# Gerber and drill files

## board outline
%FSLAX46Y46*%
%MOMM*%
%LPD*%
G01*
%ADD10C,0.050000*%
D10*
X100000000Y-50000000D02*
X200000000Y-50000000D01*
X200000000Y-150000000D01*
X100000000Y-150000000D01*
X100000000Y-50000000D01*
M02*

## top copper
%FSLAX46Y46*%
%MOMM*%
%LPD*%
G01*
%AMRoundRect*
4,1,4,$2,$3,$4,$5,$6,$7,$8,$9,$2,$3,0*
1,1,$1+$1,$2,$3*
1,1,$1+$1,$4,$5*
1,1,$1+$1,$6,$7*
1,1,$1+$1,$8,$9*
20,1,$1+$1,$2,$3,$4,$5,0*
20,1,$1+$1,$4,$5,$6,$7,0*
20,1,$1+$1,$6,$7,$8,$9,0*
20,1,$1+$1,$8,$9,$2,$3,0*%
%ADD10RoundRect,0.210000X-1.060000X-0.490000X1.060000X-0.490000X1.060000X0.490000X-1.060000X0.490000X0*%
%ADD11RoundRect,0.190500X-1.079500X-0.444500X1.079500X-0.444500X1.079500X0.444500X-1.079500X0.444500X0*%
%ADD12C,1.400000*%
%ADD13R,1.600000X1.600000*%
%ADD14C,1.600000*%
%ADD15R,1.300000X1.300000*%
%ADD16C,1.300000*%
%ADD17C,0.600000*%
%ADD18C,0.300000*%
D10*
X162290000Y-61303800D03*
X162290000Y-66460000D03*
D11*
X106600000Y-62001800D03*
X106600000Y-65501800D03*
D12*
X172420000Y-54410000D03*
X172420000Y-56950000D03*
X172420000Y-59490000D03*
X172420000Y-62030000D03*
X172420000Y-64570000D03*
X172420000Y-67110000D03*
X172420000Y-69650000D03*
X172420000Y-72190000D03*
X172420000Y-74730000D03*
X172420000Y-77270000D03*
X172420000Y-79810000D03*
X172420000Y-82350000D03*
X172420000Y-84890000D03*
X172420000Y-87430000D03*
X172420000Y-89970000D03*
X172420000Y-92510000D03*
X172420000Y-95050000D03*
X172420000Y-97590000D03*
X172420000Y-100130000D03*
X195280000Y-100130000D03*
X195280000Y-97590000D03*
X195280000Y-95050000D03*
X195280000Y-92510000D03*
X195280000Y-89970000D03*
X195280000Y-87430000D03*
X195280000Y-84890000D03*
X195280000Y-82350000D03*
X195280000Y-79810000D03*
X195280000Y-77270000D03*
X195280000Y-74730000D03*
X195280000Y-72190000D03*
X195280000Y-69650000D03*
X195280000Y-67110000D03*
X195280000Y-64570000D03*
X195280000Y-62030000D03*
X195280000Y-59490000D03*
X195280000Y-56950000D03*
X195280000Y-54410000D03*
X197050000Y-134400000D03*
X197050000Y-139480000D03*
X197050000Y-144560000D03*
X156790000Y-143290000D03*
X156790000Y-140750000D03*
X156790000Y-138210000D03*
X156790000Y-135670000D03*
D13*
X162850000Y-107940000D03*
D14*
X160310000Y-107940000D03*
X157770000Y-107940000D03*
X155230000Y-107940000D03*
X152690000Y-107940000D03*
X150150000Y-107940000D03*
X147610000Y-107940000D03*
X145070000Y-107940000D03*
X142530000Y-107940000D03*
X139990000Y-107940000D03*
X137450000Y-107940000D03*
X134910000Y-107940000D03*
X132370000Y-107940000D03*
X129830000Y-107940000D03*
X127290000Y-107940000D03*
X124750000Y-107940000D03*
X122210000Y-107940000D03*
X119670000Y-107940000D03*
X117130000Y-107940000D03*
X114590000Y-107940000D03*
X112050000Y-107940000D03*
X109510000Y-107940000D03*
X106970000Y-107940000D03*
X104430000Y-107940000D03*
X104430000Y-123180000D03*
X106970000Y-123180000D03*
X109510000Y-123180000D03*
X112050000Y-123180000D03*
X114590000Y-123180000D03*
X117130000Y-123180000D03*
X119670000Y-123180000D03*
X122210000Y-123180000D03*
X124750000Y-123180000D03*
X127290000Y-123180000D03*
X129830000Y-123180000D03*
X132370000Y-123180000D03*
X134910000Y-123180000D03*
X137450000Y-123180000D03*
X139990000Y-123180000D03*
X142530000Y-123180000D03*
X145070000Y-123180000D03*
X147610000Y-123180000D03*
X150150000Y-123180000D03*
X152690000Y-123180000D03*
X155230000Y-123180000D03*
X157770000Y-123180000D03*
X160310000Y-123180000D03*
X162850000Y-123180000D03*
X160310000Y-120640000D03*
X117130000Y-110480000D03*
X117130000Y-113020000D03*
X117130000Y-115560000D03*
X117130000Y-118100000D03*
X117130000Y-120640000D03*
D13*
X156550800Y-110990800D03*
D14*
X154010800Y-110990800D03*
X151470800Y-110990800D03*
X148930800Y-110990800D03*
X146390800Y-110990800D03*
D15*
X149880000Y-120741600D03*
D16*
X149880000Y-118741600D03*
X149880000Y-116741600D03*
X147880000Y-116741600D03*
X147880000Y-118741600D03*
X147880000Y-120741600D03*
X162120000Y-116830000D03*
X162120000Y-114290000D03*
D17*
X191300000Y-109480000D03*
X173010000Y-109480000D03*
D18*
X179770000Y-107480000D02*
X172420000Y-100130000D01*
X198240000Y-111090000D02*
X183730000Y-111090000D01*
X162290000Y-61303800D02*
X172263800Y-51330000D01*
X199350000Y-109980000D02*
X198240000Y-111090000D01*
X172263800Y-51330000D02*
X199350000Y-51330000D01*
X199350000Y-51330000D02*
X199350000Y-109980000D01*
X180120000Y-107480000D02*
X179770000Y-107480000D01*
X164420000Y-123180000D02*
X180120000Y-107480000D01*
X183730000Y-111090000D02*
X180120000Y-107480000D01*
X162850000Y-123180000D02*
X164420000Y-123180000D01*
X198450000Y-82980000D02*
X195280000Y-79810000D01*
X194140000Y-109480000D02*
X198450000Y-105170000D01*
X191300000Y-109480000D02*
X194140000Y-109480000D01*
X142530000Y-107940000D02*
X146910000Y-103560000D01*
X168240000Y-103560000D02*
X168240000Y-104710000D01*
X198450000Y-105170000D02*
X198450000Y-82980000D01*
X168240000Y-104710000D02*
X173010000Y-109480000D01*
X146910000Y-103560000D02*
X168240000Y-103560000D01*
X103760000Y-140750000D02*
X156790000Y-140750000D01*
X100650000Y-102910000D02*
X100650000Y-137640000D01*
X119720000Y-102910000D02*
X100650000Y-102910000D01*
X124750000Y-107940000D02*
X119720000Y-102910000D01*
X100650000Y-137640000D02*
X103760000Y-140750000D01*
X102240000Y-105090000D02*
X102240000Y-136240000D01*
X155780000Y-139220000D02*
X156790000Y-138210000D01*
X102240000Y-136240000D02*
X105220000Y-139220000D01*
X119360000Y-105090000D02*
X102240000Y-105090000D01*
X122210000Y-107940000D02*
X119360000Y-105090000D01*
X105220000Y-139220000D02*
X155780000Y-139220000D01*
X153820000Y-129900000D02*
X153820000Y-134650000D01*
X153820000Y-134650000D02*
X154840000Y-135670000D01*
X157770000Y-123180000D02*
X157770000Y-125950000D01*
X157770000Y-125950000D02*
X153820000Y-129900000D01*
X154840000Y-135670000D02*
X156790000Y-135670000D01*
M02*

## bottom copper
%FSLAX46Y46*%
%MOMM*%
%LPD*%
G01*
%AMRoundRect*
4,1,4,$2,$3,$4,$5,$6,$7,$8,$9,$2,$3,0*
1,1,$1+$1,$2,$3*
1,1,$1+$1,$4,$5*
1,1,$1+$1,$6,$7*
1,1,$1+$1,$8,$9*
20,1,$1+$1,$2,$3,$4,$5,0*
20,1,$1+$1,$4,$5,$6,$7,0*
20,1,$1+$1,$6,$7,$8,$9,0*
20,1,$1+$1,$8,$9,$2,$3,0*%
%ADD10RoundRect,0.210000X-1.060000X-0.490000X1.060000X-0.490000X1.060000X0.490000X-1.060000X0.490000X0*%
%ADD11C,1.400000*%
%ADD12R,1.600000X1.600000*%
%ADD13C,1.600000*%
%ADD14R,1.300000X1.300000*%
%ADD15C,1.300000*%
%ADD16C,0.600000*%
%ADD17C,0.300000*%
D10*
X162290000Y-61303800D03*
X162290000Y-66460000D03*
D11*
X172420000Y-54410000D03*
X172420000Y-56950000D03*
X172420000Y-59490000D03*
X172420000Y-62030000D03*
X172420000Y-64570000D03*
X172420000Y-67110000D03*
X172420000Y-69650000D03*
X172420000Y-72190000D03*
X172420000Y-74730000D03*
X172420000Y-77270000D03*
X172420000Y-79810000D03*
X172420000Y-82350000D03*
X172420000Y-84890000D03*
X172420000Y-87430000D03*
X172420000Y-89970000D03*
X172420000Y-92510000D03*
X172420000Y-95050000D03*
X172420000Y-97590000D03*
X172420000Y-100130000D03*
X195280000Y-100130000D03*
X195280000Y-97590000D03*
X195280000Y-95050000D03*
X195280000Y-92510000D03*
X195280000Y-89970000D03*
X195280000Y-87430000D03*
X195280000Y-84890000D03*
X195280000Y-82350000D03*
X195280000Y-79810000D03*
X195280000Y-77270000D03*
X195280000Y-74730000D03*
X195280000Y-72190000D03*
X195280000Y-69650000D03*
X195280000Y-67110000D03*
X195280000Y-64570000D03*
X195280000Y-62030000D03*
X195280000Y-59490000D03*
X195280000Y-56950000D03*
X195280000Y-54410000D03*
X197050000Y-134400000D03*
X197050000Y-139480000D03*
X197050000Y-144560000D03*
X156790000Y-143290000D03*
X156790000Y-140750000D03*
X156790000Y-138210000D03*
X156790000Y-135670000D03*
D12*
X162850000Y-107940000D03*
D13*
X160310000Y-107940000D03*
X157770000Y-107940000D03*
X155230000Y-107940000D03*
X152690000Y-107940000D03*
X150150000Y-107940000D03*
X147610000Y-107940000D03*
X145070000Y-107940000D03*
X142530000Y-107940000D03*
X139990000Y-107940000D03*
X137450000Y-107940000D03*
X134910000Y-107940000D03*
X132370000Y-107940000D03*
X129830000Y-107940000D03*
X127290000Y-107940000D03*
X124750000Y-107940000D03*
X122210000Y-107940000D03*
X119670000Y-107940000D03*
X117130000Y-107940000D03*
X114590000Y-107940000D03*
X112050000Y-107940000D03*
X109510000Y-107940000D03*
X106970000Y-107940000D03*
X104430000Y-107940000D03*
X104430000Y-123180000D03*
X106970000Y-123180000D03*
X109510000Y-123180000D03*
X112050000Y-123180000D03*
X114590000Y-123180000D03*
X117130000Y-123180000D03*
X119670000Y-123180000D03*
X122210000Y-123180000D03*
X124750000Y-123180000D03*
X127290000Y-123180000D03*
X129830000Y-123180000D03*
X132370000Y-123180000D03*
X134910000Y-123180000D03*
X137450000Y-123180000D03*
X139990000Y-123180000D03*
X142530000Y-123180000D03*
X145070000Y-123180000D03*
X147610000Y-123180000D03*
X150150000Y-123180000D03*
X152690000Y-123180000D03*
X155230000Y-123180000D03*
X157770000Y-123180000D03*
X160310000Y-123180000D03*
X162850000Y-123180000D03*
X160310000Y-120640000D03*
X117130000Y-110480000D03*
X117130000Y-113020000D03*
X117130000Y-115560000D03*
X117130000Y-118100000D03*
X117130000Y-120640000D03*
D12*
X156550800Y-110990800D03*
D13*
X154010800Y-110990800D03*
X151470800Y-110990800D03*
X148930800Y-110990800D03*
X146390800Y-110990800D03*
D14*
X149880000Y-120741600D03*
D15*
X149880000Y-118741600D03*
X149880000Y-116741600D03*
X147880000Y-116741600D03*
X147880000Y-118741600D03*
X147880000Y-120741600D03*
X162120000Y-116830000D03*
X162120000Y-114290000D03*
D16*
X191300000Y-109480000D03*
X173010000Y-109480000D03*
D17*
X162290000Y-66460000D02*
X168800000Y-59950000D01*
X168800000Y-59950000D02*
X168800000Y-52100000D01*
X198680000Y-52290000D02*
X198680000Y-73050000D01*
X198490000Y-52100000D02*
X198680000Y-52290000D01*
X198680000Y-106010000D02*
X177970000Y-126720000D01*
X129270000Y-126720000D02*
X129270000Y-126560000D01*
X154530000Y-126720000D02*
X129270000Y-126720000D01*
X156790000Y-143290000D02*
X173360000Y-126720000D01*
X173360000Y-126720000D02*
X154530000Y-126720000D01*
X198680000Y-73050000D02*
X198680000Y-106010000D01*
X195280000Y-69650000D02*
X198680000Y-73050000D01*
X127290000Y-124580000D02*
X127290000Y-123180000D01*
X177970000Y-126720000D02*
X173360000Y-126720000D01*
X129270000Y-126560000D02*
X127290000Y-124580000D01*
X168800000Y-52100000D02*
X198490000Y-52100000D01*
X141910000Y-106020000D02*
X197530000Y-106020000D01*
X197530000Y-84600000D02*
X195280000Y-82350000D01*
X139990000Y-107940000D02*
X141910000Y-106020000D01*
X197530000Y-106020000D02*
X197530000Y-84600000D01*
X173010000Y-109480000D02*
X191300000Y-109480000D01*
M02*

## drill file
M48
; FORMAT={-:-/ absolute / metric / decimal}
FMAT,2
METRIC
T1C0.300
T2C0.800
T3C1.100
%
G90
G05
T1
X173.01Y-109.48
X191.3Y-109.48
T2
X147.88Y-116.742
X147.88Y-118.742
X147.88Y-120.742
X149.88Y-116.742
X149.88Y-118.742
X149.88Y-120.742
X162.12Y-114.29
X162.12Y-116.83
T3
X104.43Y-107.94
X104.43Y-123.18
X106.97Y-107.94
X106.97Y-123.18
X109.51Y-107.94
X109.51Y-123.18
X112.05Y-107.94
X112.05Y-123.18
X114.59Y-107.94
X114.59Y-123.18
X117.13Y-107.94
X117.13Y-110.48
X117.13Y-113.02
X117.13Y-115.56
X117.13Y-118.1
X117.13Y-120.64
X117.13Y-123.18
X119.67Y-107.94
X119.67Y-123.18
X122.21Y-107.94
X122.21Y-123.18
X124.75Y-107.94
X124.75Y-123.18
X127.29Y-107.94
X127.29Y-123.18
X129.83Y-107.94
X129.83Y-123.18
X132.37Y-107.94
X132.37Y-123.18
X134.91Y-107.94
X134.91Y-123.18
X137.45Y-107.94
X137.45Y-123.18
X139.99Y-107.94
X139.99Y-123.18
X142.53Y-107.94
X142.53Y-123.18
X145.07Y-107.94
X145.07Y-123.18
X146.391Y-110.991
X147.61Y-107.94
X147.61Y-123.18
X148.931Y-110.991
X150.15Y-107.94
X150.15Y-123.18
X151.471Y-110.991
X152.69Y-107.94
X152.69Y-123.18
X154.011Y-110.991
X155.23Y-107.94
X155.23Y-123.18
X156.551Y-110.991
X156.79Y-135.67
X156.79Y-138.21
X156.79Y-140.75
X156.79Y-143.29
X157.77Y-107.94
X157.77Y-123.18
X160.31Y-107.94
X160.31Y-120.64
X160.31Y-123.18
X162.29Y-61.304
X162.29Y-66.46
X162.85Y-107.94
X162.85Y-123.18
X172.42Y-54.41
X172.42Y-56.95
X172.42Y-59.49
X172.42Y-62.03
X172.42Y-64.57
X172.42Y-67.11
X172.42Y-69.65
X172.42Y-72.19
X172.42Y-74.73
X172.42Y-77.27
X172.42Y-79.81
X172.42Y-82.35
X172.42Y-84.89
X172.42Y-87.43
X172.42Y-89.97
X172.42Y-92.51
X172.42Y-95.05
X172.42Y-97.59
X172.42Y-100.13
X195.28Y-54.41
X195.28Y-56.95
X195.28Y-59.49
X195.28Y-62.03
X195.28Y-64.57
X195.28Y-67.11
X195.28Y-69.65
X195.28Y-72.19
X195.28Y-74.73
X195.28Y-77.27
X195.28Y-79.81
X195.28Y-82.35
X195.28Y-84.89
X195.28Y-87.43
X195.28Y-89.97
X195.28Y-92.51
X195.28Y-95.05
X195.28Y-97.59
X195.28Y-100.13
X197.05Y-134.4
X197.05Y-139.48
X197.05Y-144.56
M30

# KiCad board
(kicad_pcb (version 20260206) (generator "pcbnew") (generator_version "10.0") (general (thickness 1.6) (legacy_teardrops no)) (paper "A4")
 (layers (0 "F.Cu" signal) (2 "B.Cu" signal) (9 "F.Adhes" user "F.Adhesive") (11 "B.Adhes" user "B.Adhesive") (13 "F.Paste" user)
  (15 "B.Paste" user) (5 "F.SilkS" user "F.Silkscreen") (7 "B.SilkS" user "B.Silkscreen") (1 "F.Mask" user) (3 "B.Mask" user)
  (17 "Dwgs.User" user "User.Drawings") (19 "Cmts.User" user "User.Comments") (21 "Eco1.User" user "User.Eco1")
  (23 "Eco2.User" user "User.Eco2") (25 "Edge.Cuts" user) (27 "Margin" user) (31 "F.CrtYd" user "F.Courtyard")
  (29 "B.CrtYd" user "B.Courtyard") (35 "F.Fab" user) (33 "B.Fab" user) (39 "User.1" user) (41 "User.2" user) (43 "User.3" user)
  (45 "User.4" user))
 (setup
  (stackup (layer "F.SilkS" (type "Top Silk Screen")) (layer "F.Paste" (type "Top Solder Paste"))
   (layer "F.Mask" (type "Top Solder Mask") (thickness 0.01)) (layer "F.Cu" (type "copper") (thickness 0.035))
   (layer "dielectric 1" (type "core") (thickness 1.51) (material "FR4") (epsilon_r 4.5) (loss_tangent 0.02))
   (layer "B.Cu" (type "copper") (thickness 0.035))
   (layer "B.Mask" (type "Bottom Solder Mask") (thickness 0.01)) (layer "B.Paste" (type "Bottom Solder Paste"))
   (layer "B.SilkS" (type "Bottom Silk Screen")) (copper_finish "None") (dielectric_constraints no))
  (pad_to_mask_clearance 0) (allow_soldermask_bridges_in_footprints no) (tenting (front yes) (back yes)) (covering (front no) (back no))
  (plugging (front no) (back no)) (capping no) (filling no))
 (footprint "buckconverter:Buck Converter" (layer "F.Cu") (at 102.6 58.0018)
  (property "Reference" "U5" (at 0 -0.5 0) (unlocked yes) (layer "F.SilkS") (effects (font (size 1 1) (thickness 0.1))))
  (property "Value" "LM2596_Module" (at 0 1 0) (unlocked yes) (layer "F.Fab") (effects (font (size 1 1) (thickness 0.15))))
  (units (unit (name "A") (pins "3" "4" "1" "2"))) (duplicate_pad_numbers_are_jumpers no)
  (pad "1" thru_hole roundrect (at 59.69 3.302) (size 2.54 1.4) (drill 1.1) (layers "*.Cu" "*.Mask") (remove_unused_layers no)
   (roundrect_rratio 0.15) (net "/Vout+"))
  (pad "2" thru_hole roundrect (at 59.69 8.4582) (size 2.54 1.4) (drill 1.1) (layers "*.Cu" "*.Mask") (remove_unused_layers no)
   (roundrect_rratio 0.15) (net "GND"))
  (pad "3" smd roundrect (at 4 4) (size 2.54 1.27) (layers "F.Cu" "F.Mask" "F.Paste") (roundrect_rratio 0.15) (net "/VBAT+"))
  (pad "4" smd roundrect (at 4 7.5) (size 2.54 1.27) (layers "F.Cu" "F.Mask" "F.Paste") (roundrect_rratio 0.15) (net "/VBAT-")))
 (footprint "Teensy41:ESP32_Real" (layer "F.Cu") (at 172.42 54.41)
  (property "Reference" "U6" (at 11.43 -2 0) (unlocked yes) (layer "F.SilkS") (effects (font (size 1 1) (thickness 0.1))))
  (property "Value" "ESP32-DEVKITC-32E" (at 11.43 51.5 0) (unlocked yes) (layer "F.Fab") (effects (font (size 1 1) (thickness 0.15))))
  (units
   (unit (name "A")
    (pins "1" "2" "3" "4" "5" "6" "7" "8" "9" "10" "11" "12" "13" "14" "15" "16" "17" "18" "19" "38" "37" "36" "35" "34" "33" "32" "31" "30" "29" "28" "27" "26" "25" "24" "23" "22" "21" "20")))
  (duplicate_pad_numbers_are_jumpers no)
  (pad "1" thru_hole circle (at 0 0) (size 1.4 1.4) (drill 1.1) (layers "*.Cu" "*.Mask") (remove_unused_layers no)
   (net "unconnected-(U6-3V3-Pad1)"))
  (pad "2" thru_hole circle (at 0 2.54) (size 1.4 1.4) (drill 1.1) (layers "*.Cu" "*.Mask") (remove_unused_layers no)
   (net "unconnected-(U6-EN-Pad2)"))
  (pad "3" thru_hole circle (at 0 5.08) (size 1.4 1.4) (drill 1.1) (layers "*.Cu" "*.Mask") (remove_unused_layers no)
   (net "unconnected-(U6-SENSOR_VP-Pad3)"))
  (pad "4" thru_hole circle (at 0 7.62) (size 1.4 1.4) (drill 1.1) (layers "*.Cu" "*.Mask") (remove_unused_layers no)
   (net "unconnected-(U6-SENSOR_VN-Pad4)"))
  (pad "5" thru_hole circle (at 0 10.16) (size 1.4 1.4) (drill 1.1) (layers "*.Cu" "*.Mask") (remove_unused_layers no)
   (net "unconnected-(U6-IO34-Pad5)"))
  (pad "6" thru_hole circle (at 0 12.7) (size 1.4 1.4) (drill 1.1) (layers "*.Cu" "*.Mask") (remove_unused_layers no)
   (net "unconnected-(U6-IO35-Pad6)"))
  (pad "7" thru_hole circle (at 0 15.24) (size 1.4 1.4) (drill 1.1) (layers "*.Cu" "*.Mask") (remove_unused_layers no)
   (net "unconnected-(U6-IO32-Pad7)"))
  (pad "8" thru_hole circle (at 0 17.78) (size 1.4 1.4) (drill 1.1) (layers "*.Cu" "*.Mask") (remove_unused_layers no)
   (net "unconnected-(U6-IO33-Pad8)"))
  (pad "9" thru_hole circle (at 0 20.32) (size 1.4 1.4) (drill 1.1) (layers "*.Cu" "*.Mask") (remove_unused_layers no)
   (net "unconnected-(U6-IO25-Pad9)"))
  (pad "10" thru_hole circle (at 0 22.86) (size 1.4 1.4) (drill 1.1) (layers "*.Cu" "*.Mask") (remove_unused_layers no)
   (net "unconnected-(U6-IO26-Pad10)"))
  (pad "11" thru_hole circle (at 0 25.4) (size 1.4 1.4) (drill 1.1) (layers "*.Cu" "*.Mask") (remove_unused_layers no)
   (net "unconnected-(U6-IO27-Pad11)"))
  (pad "12" thru_hole circle (at 0 27.94) (size 1.4 1.4) (drill 1.1) (layers "*.Cu" "*.Mask") (remove_unused_layers no)
   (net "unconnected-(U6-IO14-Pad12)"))
  (pad "13" thru_hole circle (at 0 30.48) (size 1.4 1.4) (drill 1.1) (layers "*.Cu" "*.Mask") (remove_unused_layers no)
   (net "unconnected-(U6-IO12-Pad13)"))
  (pad "14" thru_hole circle (at 0 33.02) (size 1.4 1.4) (drill 1.1) (layers "*.Cu" "*.Mask") (remove_unused_layers no)
   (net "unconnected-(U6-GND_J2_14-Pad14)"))
  (pad "15" thru_hole circle (at 0 35.56) (size 1.4 1.4) (drill 1.1) (layers "*.Cu" "*.Mask") (remove_unused_layers no)
   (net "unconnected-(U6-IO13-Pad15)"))
  (pad "16" thru_hole circle (at 0 38.1) (size 1.4 1.4) (drill 1.1) (layers "*.Cu" "*.Mask") (remove_unused_layers no)
   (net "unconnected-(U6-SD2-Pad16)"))
  (pad "17" thru_hole circle (at 0 40.64) (size 1.4 1.4) (drill 1.1) (layers "*.Cu" "*.Mask") (remove_unused_layers no)
   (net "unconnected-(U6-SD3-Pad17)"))
  (pad "18" thru_hole circle (at 0 43.18) (size 1.4 1.4) (drill 1.1) (layers "*.Cu" "*.Mask") (remove_unused_layers no)
   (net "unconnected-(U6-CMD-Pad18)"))
  (pad "19" thru_hole circle (at 0 45.72) (size 1.4 1.4) (drill 1.1) (layers "*.Cu" "*.Mask") (remove_unused_layers no) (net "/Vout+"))
  (pad "20" thru_hole circle (at 22.86 45.72) (size 1.4 1.4) (drill 1.1) (layers "*.Cu" "*.Mask") (remove_unused_layers no)
   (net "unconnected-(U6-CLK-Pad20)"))
  (pad "21" thru_hole circle (at 22.86 43.18) (size 1.4 1.4) (drill 1.1) (layers "*.Cu" "*.Mask") (remove_unused_layers no)
   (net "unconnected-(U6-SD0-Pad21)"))
  (pad "22" thru_hole circle (at 22.86 40.64) (size 1.4 1.4) (drill 1.1) (layers "*.Cu" "*.Mask") (remove_unused_layers no)
   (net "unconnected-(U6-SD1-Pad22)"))
  (pad "23" thru_hole circle (at 22.86 38.1) (size 1.4 1.4) (drill 1.1) (layers "*.Cu" "*.Mask") (remove_unused_layers no)
   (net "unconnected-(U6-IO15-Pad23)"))
  (pad "24" thru_hole circle (at 22.86 35.56) (size 1.4 1.4) (drill 1.1) (layers "*.Cu" "*.Mask") (remove_unused_layers no)
   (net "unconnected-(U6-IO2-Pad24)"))
  (pad "25" thru_hole circle (at 22.86 33.02) (size 1.4 1.4) (drill 1.1) (layers "*.Cu" "*.Mask") (remove_unused_layers no)
   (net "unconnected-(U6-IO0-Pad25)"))
  (pad "26" thru_hole circle (at 22.86 30.48) (size 1.4 1.4) (drill 1.1) (layers "*.Cu" "*.Mask") (remove_unused_layers no)
   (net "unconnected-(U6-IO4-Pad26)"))
  (pad "27" thru_hole circle (at 22.86 27.94) (size 1.4 1.4) (drill 1.1) (layers "*.Cu" "*.Mask") (remove_unused_layers no)
   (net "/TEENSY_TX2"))
  (pad "28" thru_hole circle (at 22.86 25.4) (size 1.4 1.4) (drill 1.1) (layers "*.Cu" "*.Mask") (remove_unused_layers no)
   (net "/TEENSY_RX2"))
  (pad "29" thru_hole circle (at 22.86 22.86) (size 1.4 1.4) (drill 1.1) (layers "*.Cu" "*.Mask") (remove_unused_layers no)
   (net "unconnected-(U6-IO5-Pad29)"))
  (pad "30" thru_hole circle (at 22.86 20.32) (size 1.4 1.4) (drill 1.1) (layers "*.Cu" "*.Mask") (remove_unused_layers no)
   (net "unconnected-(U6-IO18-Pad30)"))
  (pad "31" thru_hole circle (at 22.86 17.78) (size 1.4 1.4) (drill 1.1) (layers "*.Cu" "*.Mask") (remove_unused_layers no)
   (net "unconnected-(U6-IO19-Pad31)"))
  (pad "32" thru_hole circle (at 22.86 15.24) (size 1.4 1.4) (drill 1.1) (layers "*.Cu" "*.Mask") (remove_unused_layers no) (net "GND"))
  (pad "33" thru_hole circle (at 22.86 12.7) (size 1.4 1.4) (drill 1.1) (layers "*.Cu" "*.Mask") (remove_unused_layers no)
   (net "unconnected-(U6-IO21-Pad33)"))
  (pad "34" thru_hole circle (at 22.86 10.16) (size 1.4 1.4) (drill 1.1) (layers "*.Cu" "*.Mask") (remove_unused_layers no)
   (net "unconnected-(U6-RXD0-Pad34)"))
  (pad "35" thru_hole circle (at 22.86 7.62) (size 1.4 1.4) (drill 1.1) (layers "*.Cu" "*.Mask") (remove_unused_layers no)
   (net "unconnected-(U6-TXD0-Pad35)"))
  (pad "36" thru_hole circle (at 22.86 5.08) (size 1.4 1.4) (drill 1.1) (layers "*.Cu" "*.Mask") (remove_unused_layers no)
   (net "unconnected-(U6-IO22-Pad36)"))
  (pad "37" thru_hole circle (at 22.86 2.54) (size 1.4 1.4) (drill 1.1) (layers "*.Cu" "*.Mask") (remove_unused_layers no)
   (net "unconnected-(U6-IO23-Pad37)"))
  (pad "38" thru_hole circle (at 22.86 0) (size 1.4 1.4) (drill 1.1) (layers "*.Cu" "*.Mask") (remove_unused_layers no)
   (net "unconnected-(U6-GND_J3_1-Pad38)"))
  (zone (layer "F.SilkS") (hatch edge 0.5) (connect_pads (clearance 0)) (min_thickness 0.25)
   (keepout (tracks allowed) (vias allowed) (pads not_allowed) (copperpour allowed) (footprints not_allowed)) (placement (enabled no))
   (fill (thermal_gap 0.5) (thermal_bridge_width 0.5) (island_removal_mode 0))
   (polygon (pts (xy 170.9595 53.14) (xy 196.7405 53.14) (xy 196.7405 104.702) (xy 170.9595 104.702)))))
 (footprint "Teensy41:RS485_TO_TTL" (layer "F.Cu") (at 155.52 131.86)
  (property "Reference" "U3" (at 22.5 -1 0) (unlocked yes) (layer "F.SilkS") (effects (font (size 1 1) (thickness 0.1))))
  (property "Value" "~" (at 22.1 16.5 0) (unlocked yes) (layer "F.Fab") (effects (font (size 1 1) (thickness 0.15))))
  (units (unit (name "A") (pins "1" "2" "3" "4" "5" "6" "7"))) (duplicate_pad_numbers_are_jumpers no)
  (pad "1" thru_hole circle (at 41.53 2.54) (size 1.4 1.4) (drill 1.1) (layers "*.Cu" "*.Mask") (remove_unused_layers no)
   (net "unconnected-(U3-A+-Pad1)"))
  (pad "2" thru_hole circle (at 41.53 7.62) (size 1.4 1.4) (drill 1.1) (layers "*.Cu" "*.Mask") (remove_unused_layers no)
   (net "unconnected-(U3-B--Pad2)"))
  (pad "3" thru_hole circle (at 41.53 12.7) (size 1.4 1.4) (drill 1.1) (layers "*.Cu" "*.Mask") (remove_unused_layers no)
   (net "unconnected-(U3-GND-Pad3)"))
  (pad "4" thru_hole circle (at 1.27 11.43) (size 1.4 1.4) (drill 1.1) (layers "*.Cu" "*.Mask") (remove_unused_layers no) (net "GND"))
  (pad "5" thru_hole circle (at 1.27 8.89) (size 1.4 1.4) (drill 1.1) (layers "*.Cu" "*.Mask") (remove_unused_layers no) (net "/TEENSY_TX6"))
  (pad "6" thru_hole circle (at 1.27 6.35) (size 1.4 1.4) (drill 1.1) (layers "*.Cu" "*.Mask") (remove_unused_layers no) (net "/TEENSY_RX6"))
  (pad "7" thru_hole circle (at 1.27 3.81) (size 1.4 1.4) (drill 1.1) (layers "*.Cu" "*.Mask") (remove_unused_layers no) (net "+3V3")))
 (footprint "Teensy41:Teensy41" (layer "F.Cu") (at 133.64 115.56 180)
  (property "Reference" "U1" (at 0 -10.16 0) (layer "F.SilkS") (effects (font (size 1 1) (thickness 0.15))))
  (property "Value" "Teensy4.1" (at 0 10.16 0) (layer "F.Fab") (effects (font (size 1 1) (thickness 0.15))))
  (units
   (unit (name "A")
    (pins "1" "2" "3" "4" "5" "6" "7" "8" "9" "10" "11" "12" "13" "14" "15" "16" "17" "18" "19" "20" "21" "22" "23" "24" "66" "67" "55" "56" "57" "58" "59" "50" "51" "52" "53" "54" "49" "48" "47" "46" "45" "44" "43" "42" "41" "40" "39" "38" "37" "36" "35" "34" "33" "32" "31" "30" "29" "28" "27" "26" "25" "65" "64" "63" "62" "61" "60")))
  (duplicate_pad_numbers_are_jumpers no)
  (pad "1" thru_hole rect (at -29.21 7.62 180) (size 1.6 1.6) (drill 1.1) (layers "*.Cu" "*.Mask") (remove_unused_layers no)
   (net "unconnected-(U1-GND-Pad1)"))
  (pad "2" thru_hole circle (at -26.67 7.62 180) (size 1.6 1.6) (drill 1.1) (layers "*.Cu" "*.Mask") (remove_unused_layers no)
   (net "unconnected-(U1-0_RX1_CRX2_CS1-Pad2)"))
  (pad "3" thru_hole circle (at -24.13 7.62 180) (size 1.6 1.6) (drill 1.1) (layers "*.Cu" "*.Mask") (remove_unused_layers no)
   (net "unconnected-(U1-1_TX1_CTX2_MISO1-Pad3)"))
  (pad "4" thru_hole circle (at -21.59 7.62 180) (size 1.6 1.6) (drill 1.1) (layers "*.Cu" "*.Mask") (remove_unused_layers no)
   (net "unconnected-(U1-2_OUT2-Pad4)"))
  (pad "5" thru_hole circle (at -19.05 7.62 180) (size 1.6 1.6) (drill 1.1) (layers "*.Cu" "*.Mask") (remove_unused_layers no)
   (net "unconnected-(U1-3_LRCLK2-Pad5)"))
  (pad "6" thru_hole circle (at -16.51 7.62 180) (size 1.6 1.6) (drill 1.1) (layers "*.Cu" "*.Mask") (remove_unused_layers no)
   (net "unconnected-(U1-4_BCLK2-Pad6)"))
  (pad "7" thru_hole circle (at -13.97 7.62 180) (size 1.6 1.6) (drill 1.1) (layers "*.Cu" "*.Mask") (remove_unused_layers no)
   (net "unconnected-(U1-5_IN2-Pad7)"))
  (pad "8" thru_hole circle (at -11.43 7.62 180) (size 1.6 1.6) (drill 1.1) (layers "*.Cu" "*.Mask") (remove_unused_layers no)
   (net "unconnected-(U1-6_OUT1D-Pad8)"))
  (pad "9" thru_hole circle (at -8.89 7.62 180) (size 1.6 1.6) (drill 1.1) (layers "*.Cu" "*.Mask") (remove_unused_layers no)
   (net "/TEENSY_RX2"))
  (pad "10" thru_hole circle (at -6.35 7.62 180) (size 1.6 1.6) (drill 1.1) (layers "*.Cu" "*.Mask") (remove_unused_layers no)
   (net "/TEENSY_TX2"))
  (pad "11" thru_hole circle (at -3.81 7.62 180) (size 1.6 1.6) (drill 1.1) (layers "*.Cu" "*.Mask") (remove_unused_layers no)
   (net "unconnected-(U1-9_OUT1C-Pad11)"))
  (pad "12" thru_hole circle (at -1.27 7.62 180) (size 1.6 1.6) (drill 1.1) (layers "*.Cu" "*.Mask") (remove_unused_layers no)
   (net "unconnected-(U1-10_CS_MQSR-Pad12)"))
  (pad "13" thru_hole circle (at 1.27 7.62 180) (size 1.6 1.6) (drill 1.1) (layers "*.Cu" "*.Mask") (remove_unused_layers no)
   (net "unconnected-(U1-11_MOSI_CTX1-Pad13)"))
  (pad "14" thru_hole circle (at 3.81 7.62 180) (size 1.6 1.6) (drill 1.1) (layers "*.Cu" "*.Mask") (remove_unused_layers no)
   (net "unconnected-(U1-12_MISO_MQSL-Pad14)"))
  (pad "15" thru_hole circle (at 6.35 7.62 180) (size 1.6 1.6) (drill 1.1) (layers "*.Cu" "*.Mask") (remove_unused_layers no)
   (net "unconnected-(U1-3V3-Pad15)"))
  (pad "16" thru_hole circle (at 8.89 7.62 180) (size 1.6 1.6) (drill 1.1) (layers "*.Cu" "*.Mask") (remove_unused_layers no)
   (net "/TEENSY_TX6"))
  (pad "17" thru_hole circle (at 11.43 7.62 180) (size 1.6 1.6) (drill 1.1) (layers "*.Cu" "*.Mask") (remove_unused_layers no)
   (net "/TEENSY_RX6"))
  (pad "18" thru_hole circle (at 13.97 7.62 180) (size 1.6 1.6) (drill 1.1) (layers "*.Cu" "*.Mask") (remove_unused_layers no)
   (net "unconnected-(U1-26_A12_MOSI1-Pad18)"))
  (pad "19" thru_hole circle (at 16.51 7.62 180) (size 1.6 1.6) (drill 1.1) (layers "*.Cu" "*.Mask") (remove_unused_layers no)
   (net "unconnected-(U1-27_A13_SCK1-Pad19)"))
  (pad "20" thru_hole circle (at 19.05 7.62 180) (size 1.6 1.6) (drill 1.1) (layers "*.Cu" "*.Mask") (remove_unused_layers no)
   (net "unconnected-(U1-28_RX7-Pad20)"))
  (pad "21" thru_hole circle (at 21.59 7.62 180) (size 1.6 1.6) (drill 1.1) (layers "*.Cu" "*.Mask") (remove_unused_layers no)
   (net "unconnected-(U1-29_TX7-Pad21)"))
  (pad "22" thru_hole circle (at 24.13 7.62 180) (size 1.6 1.6) (drill 1.1) (layers "*.Cu" "*.Mask") (remove_unused_layers no)
   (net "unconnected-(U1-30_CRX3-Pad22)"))
  (pad "23" thru_hole circle (at 26.67 7.62 180) (size 1.6 1.6) (drill 1.1) (layers "*.Cu" "*.Mask") (remove_unused_layers no)
   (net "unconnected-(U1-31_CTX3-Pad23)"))
  (pad "24" thru_hole circle (at 29.21 7.62 180) (size 1.6 1.6) (drill 1.1) (layers "*.Cu" "*.Mask") (remove_unused_layers no)
   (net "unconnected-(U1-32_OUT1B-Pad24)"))
  (pad "25" thru_hole circle (at 29.21 -7.62 180) (size 1.6 1.6) (drill 1.1) (layers "*.Cu" "*.Mask") (remove_unused_layers no)
   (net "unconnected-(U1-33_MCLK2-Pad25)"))
  (pad "26" thru_hole circle (at 26.67 -7.62 180) (size 1.6 1.6) (drill 1.1) (layers "*.Cu" "*.Mask") (remove_unused_layers no)
   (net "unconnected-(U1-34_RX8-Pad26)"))
  (pad "27" thru_hole circle (at 24.13 -7.62 180) (size 1.6 1.6) (drill 1.1) (layers "*.Cu" "*.Mask") (remove_unused_layers no)
   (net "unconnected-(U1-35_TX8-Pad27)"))
  (pad "28" thru_hole circle (at 21.59 -7.62 180) (size 1.6 1.6) (drill 1.1) (layers "*.Cu" "*.Mask") (remove_unused_layers no)
   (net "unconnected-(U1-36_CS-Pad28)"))
  (pad "29" thru_hole circle (at 19.05 -7.62 180) (size 1.6 1.6) (drill 1.1) (layers "*.Cu" "*.Mask") (remove_unused_layers no)
   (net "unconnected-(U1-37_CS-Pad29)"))
  (pad "30" thru_hole circle (at 16.51 -7.62 180) (size 1.6 1.6) (drill 1.1) (layers "*.Cu" "*.Mask") (remove_unused_layers no)
   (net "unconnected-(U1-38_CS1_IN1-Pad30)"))
  (pad "31" thru_hole circle (at 13.97 -7.62 180) (size 1.6 1.6) (drill 1.1) (layers "*.Cu" "*.Mask") (remove_unused_layers no)
   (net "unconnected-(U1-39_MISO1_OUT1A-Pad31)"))
  (pad "32" thru_hole circle (at 11.43 -7.62 180) (size 1.6 1.6) (drill 1.1) (layers "*.Cu" "*.Mask") (remove_unused_layers no)
   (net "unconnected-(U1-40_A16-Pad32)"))
  (pad "33" thru_hole circle (at 8.89 -7.62 180) (size 1.6 1.6) (drill 1.1) (layers "*.Cu" "*.Mask") (remove_unused_layers no)
   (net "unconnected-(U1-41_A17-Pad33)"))
  (pad "34" thru_hole circle (at 6.35 -7.62 180) (size 1.6 1.6) (drill 1.1) (layers "*.Cu" "*.Mask") (remove_unused_layers no) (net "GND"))
  (pad "35" thru_hole circle (at 3.81 -7.62 180) (size 1.6 1.6) (drill 1.1) (layers "*.Cu" "*.Mask") (remove_unused_layers no)
   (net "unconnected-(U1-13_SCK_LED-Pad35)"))
  (pad "36" thru_hole circle (at 1.27 -7.62 180) (size 1.6 1.6) (drill 1.1) (layers "*.Cu" "*.Mask") (remove_unused_layers no)
   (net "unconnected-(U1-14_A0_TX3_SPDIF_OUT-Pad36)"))
  (pad "37" thru_hole circle (at -1.27 -7.62 180) (size 1.6 1.6) (drill 1.1) (layers "*.Cu" "*.Mask") (remove_unused_layers no)
   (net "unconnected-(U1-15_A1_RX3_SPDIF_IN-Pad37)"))
  (pad "38" thru_hole circle (at -3.81 -7.62 180) (size 1.6 1.6) (drill 1.1) (layers "*.Cu" "*.Mask") (remove_unused_layers no)
   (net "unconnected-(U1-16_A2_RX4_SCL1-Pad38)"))
  (pad "39" thru_hole circle (at -6.35 -7.62 180) (size 1.6 1.6) (drill 1.1) (layers "*.Cu" "*.Mask") (remove_unused_layers no)
   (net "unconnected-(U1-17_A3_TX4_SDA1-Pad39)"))
  (pad "40" thru_hole circle (at -8.89 -7.62 180) (size 1.6 1.6) (drill 1.1) (layers "*.Cu" "*.Mask") (remove_unused_layers no)
   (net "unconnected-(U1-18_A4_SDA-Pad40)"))
  (pad "41" thru_hole circle (at -11.43 -7.62 180) (size 1.6 1.6) (drill 1.1) (layers "*.Cu" "*.Mask") (remove_unused_layers no)
   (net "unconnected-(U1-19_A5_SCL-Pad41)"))
  (pad "42" thru_hole circle (at -13.97 -7.62 180) (size 1.6 1.6) (drill 1.1) (layers "*.Cu" "*.Mask") (remove_unused_layers no)
   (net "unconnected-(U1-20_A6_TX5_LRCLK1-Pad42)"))
  (pad "43" thru_hole circle (at -16.51 -7.62 180) (size 1.6 1.6) (drill 1.1) (layers "*.Cu" "*.Mask") (remove_unused_layers no)
   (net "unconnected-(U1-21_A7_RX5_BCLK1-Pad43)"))
  (pad "44" thru_hole circle (at -19.05 -7.62 180) (size 1.6 1.6) (drill 1.1) (layers "*.Cu" "*.Mask") (remove_unused_layers no)
   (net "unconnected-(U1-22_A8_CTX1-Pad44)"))
  (pad "45" thru_hole circle (at -21.59 -7.62 180) (size 1.6 1.6) (drill 1.1) (layers "*.Cu" "*.Mask") (remove_unused_layers no)
   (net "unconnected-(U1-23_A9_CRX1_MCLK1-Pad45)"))
  (pad "46" thru_hole circle (at -24.13 -7.62 180) (size 1.6 1.6) (drill 1.1) (layers "*.Cu" "*.Mask") (remove_unused_layers no)
   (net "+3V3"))
  (pad "47" thru_hole circle (at -26.67 -7.62 180) (size 1.6 1.6) (drill 1.1) (layers "*.Cu" "*.Mask") (remove_unused_layers no)
   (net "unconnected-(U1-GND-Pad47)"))
  (pad "48" thru_hole circle (at -29.21 -7.62 180) (size 1.6 1.6) (drill 1.1) (layers "*.Cu" "*.Mask") (remove_unused_layers no)
   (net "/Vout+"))
  (pad "49" thru_hole circle (at -26.67 -5.08 180) (size 1.6 1.6) (drill 1.1) (layers "*.Cu" "*.Mask") (remove_unused_layers no)
   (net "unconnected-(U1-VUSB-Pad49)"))
  (pad "50" thru_hole circle (at 16.51 5.08 180) (size 1.6 1.6) (drill 1.1) (layers "*.Cu" "*.Mask") (remove_unused_layers no)
   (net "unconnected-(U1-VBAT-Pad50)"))
  (pad "51" thru_hole circle (at 16.51 2.54 180) (size 1.6 1.6) (drill 1.1) (layers "*.Cu" "*.Mask") (remove_unused_layers no)
   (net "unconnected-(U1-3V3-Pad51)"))
  (pad "52" thru_hole circle (at 16.51 0 180) (size 1.6 1.6) (drill 1.1) (layers "*.Cu" "*.Mask") (remove_unused_layers no)
   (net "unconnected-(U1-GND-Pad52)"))
  (pad "53" thru_hole circle (at 16.51 -2.54 180) (size 1.6 1.6) (drill 1.1) (layers "*.Cu" "*.Mask") (remove_unused_layers no)
   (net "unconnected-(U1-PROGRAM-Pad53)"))
  (pad "54" thru_hole circle (at 16.51 -5.08 180) (size 1.6 1.6) (drill 1.1) (layers "*.Cu" "*.Mask") (remove_unused_layers no)
   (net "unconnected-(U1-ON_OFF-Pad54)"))
  (pad "55" thru_hole rect (at -22.9108 4.5692 180) (size 1.6 1.6) (drill 1.1) (layers "*.Cu" "*.Mask") (remove_unused_layers no)
   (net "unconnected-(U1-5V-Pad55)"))
  (pad "56" thru_hole circle (at -20.3708 4.5692 180) (size 1.6 1.6) (drill 1.1) (layers "*.Cu" "*.Mask") (remove_unused_layers no)
   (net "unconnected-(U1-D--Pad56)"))
  (pad "57" thru_hole circle (at -17.8308 4.5692 180) (size 1.6 1.6) (drill 1.1) (layers "*.Cu" "*.Mask") (remove_unused_layers no)
   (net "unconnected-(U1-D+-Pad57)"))
  (pad "58" thru_hole circle (at -15.2908 4.5692 180) (size 1.6 1.6) (drill 1.1) (layers "*.Cu" "*.Mask") (remove_unused_layers no)
   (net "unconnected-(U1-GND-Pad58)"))
  (pad "59" thru_hole circle (at -12.7508 4.5692 180) (size 1.6 1.6) (drill 1.1) (layers "*.Cu" "*.Mask") (remove_unused_layers no)
   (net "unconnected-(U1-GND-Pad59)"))
  (pad "60" thru_hole rect (at -16.24 -5.1816 180) (size 1.3 1.3) (drill 0.8) (layers "*.Cu" "*.Mask") (remove_unused_layers no)
   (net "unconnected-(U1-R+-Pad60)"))
  (pad "61" thru_hole circle (at -16.24 -3.1816 180) (size 1.3 1.3) (drill 0.8) (layers "*.Cu" "*.Mask") (remove_unused_layers no)
   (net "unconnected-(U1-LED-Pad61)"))
  (pad "62" thru_hole circle (at -16.24 -1.1816 180) (size 1.3 1.3) (drill 0.8) (layers "*.Cu" "*.Mask") (remove_unused_layers no)
   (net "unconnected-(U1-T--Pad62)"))
  (pad "63" thru_hole circle (at -14.24 -1.1816 180) (size 1.3 1.3) (drill 0.8) (layers "*.Cu" "*.Mask") (remove_unused_layers no)
   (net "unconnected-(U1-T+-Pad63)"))
  (pad "64" thru_hole circle (at -14.24 -3.1816 180) (size 1.3 1.3) (drill 0.8) (layers "*.Cu" "*.Mask") (remove_unused_layers no)
   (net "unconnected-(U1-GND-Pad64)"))
  (pad "65" thru_hole circle (at -14.24 -5.1816 180) (size 1.3 1.3) (drill 0.8) (layers "*.Cu" "*.Mask") (remove_unused_layers no)
   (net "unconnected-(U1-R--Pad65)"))
  (pad "66" thru_hole circle (at -28.48 -1.27 180) (size 1.3 1.3) (drill 0.8) (layers "*.Cu" "*.Mask") (remove_unused_layers no)
   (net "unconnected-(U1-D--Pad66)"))
  (pad "67" thru_hole circle (at -28.48 1.27 180) (size 1.3 1.3) (drill 0.8) (layers "*.Cu" "*.Mask") (remove_unused_layers no)
   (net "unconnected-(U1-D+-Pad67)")))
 (gr_rect (start 100 50) (end 200 150) (stroke (width 0.05) (type default)) (fill no) (layer "Edge.Cuts"))
 (segment (start 179.77 107.48) (end 172.42 100.13) (width 0.3) (layer "F.Cu") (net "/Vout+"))
 (segment (start 198.24 111.09) (end 183.73 111.09) (width 0.3) (layer "F.Cu") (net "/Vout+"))
 (segment (start 162.29 61.3038) (end 172.2638 51.33) (width 0.3) (layer "F.Cu") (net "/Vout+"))
 (segment (start 199.35 109.98) (end 198.24 111.09) (width 0.3) (layer "F.Cu") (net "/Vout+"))
 (segment (start 172.2638 51.33) (end 199.35 51.33) (width 0.3) (layer "F.Cu") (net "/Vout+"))
 (segment (start 199.35 51.33) (end 199.35 109.98) (width 0.3) (layer "F.Cu") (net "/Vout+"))
 (segment (start 180.12 107.48) (end 179.77 107.48) (width 0.3) (layer "F.Cu") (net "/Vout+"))
 (segment (start 164.42 123.18) (end 180.12 107.48) (width 0.3) (layer "F.Cu") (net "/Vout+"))
 (segment (start 183.73 111.09) (end 180.12 107.48) (width 0.3) (layer "F.Cu") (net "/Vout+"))
 (segment (start 162.85 123.18) (end 164.42 123.18) (width 0.3) (layer "F.Cu") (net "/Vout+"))
 (segment (start 162.29 66.46) (end 168.8 59.95) (width 0.3) (layer "B.Cu") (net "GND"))
 (segment (start 168.8 59.95) (end 168.8 52.1) (width 0.3) (layer "B.Cu") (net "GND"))
 (segment (start 198.68 52.29) (end 198.68 73.05) (width 0.3) (layer "B.Cu") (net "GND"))
 (segment (start 198.49 52.1) (end 198.68 52.29) (width 0.3) (layer "B.Cu") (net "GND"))
 (segment (start 198.68 106.01) (end 177.97 126.72) (width 0.3) (layer "B.Cu") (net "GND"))
 (segment (start 129.27 126.72) (end 129.27 126.56) (width 0.3) (layer "B.Cu") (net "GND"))
 (segment (start 154.53 126.72) (end 129.27 126.72) (width 0.3) (layer "B.Cu") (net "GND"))
 (segment (start 156.79 143.29) (end 173.36 126.72) (width 0.3) (layer "B.Cu") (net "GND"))
 (segment (start 173.36 126.72) (end 154.53 126.72) (width 0.3) (layer "B.Cu") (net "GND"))
 (segment (start 198.68 73.05) (end 198.68 106.01) (width 0.3) (layer "B.Cu") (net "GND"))
 (segment (start 195.28 69.65) (end 198.68 73.05) (width 0.3) (layer "B.Cu") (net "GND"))
 (segment (start 127.29 124.58) (end 127.29 123.18) (width 0.3) (layer "B.Cu") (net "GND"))
 (segment (start 177.97 126.72) (end 173.36 126.72) (width 0.3) (layer "B.Cu") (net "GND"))
 (segment (start 129.27 126.56) (end 127.29 124.58) (width 0.3) (layer "B.Cu") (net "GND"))
 (segment (start 168.8 52.1) (end 198.49 52.1) (width 0.3) (layer "B.Cu") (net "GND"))
 (segment (start 141.91 106.02) (end 197.53 106.02) (width 0.3) (layer "B.Cu") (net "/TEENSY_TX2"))
 (segment (start 197.53 84.6) (end 195.28 82.35) (width 0.3) (layer "B.Cu") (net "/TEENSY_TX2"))
 (segment (start 139.99 107.94) (end 141.91 106.02) (width 0.3) (layer "B.Cu") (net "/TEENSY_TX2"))
 (segment (start 197.53 106.02) (end 197.53 84.6) (width 0.3) (layer "B.Cu") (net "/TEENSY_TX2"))
 (segment (start 198.45 82.98) (end 195.28 79.81) (width 0.3) (layer "F.Cu") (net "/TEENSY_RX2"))
 (segment (start 194.14 109.48) (end 198.45 105.17) (width 0.3) (layer "F.Cu") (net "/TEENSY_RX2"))
 (segment (start 191.3 109.48) (end 194.14 109.48) (width 0.3) (layer "F.Cu") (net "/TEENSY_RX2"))
 (segment (start 142.53 107.94) (end 146.91 103.56) (width 0.3) (layer "F.Cu") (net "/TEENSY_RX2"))
 (segment (start 168.24 103.56) (end 168.24 104.71) (width 0.3) (layer "F.Cu") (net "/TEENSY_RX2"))
 (segment (start 198.45 105.17) (end 198.45 82.98) (width 0.3) (layer "F.Cu") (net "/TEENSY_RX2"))
 (segment (start 168.24 104.71) (end 173.01 109.48) (width 0.3) (layer "F.Cu") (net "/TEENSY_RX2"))
 (segment (start 146.91 103.56) (end 168.24 103.56) (width 0.3) (layer "F.Cu") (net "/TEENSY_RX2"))
 (via (at 191.3 109.48) (size 0.6) (drill 0.3) (layers "F.Cu" "B.Cu") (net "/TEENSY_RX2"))
 (via (at 173.01 109.48) (size 0.6) (drill 0.3) (layers "F.Cu" "B.Cu") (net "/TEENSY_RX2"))
 (segment (start 173.01 109.48) (end 191.3 109.48) (width 0.3) (layer "B.Cu") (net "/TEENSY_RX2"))
 (segment (start 103.76 140.75) (end 156.79 140.75) (width 0.3) (layer "F.Cu") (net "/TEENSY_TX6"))
 (segment (start 100.65 102.91) (end 100.65 137.64) (width 0.3) (layer "F.Cu") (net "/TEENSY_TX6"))
 (segment (start 119.72 102.91) (end 100.65 102.91) (width 0.3) (layer "F.Cu") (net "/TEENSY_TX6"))
 (segment (start 124.75 107.94) (end 119.72 102.91) (width 0.3) (layer "F.Cu") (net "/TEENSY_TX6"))
 (segment (start 100.65 137.64) (end 103.76 140.75) (width 0.3) (layer "F.Cu") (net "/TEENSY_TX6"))
 (segment (start 102.24 105.09) (end 102.24 136.24) (width 0.3) (layer "F.Cu") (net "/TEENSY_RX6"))
 (segment (start 155.78 139.22) (end 156.79 138.21) (width 0.3) (layer "F.Cu") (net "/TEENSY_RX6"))
 (segment (start 102.24 136.24) (end 105.22 139.22) (width 0.3) (layer "F.Cu") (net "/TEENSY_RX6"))
 (segment (start 119.36 105.09) (end 102.24 105.09) (width 0.3) (layer "F.Cu") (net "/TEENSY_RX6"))
 (segment (start 122.21 107.94) (end 119.36 105.09) (width 0.3) (layer "F.Cu") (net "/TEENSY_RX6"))
 (segment (start 105.22 139.22) (end 155.78 139.22) (width 0.3) (layer "F.Cu") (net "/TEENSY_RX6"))
 (segment (start 153.82 129.9) (end 153.82 134.65) (width 0.3) (layer "F.Cu") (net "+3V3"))
 (segment (start 153.82 134.65) (end 154.84 135.67) (width 0.3) (layer "F.Cu") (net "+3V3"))
 (segment (start 157.77 123.18) (end 157.77 125.95) (width 0.3) (layer "F.Cu") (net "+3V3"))
 (segment (start 157.77 125.95) (end 153.82 129.9) (width 0.3) (layer "F.Cu") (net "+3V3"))
 (segment (start 154.84 135.67) (end 156.79 135.67) (width 0.3) (layer "F.Cu") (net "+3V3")))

